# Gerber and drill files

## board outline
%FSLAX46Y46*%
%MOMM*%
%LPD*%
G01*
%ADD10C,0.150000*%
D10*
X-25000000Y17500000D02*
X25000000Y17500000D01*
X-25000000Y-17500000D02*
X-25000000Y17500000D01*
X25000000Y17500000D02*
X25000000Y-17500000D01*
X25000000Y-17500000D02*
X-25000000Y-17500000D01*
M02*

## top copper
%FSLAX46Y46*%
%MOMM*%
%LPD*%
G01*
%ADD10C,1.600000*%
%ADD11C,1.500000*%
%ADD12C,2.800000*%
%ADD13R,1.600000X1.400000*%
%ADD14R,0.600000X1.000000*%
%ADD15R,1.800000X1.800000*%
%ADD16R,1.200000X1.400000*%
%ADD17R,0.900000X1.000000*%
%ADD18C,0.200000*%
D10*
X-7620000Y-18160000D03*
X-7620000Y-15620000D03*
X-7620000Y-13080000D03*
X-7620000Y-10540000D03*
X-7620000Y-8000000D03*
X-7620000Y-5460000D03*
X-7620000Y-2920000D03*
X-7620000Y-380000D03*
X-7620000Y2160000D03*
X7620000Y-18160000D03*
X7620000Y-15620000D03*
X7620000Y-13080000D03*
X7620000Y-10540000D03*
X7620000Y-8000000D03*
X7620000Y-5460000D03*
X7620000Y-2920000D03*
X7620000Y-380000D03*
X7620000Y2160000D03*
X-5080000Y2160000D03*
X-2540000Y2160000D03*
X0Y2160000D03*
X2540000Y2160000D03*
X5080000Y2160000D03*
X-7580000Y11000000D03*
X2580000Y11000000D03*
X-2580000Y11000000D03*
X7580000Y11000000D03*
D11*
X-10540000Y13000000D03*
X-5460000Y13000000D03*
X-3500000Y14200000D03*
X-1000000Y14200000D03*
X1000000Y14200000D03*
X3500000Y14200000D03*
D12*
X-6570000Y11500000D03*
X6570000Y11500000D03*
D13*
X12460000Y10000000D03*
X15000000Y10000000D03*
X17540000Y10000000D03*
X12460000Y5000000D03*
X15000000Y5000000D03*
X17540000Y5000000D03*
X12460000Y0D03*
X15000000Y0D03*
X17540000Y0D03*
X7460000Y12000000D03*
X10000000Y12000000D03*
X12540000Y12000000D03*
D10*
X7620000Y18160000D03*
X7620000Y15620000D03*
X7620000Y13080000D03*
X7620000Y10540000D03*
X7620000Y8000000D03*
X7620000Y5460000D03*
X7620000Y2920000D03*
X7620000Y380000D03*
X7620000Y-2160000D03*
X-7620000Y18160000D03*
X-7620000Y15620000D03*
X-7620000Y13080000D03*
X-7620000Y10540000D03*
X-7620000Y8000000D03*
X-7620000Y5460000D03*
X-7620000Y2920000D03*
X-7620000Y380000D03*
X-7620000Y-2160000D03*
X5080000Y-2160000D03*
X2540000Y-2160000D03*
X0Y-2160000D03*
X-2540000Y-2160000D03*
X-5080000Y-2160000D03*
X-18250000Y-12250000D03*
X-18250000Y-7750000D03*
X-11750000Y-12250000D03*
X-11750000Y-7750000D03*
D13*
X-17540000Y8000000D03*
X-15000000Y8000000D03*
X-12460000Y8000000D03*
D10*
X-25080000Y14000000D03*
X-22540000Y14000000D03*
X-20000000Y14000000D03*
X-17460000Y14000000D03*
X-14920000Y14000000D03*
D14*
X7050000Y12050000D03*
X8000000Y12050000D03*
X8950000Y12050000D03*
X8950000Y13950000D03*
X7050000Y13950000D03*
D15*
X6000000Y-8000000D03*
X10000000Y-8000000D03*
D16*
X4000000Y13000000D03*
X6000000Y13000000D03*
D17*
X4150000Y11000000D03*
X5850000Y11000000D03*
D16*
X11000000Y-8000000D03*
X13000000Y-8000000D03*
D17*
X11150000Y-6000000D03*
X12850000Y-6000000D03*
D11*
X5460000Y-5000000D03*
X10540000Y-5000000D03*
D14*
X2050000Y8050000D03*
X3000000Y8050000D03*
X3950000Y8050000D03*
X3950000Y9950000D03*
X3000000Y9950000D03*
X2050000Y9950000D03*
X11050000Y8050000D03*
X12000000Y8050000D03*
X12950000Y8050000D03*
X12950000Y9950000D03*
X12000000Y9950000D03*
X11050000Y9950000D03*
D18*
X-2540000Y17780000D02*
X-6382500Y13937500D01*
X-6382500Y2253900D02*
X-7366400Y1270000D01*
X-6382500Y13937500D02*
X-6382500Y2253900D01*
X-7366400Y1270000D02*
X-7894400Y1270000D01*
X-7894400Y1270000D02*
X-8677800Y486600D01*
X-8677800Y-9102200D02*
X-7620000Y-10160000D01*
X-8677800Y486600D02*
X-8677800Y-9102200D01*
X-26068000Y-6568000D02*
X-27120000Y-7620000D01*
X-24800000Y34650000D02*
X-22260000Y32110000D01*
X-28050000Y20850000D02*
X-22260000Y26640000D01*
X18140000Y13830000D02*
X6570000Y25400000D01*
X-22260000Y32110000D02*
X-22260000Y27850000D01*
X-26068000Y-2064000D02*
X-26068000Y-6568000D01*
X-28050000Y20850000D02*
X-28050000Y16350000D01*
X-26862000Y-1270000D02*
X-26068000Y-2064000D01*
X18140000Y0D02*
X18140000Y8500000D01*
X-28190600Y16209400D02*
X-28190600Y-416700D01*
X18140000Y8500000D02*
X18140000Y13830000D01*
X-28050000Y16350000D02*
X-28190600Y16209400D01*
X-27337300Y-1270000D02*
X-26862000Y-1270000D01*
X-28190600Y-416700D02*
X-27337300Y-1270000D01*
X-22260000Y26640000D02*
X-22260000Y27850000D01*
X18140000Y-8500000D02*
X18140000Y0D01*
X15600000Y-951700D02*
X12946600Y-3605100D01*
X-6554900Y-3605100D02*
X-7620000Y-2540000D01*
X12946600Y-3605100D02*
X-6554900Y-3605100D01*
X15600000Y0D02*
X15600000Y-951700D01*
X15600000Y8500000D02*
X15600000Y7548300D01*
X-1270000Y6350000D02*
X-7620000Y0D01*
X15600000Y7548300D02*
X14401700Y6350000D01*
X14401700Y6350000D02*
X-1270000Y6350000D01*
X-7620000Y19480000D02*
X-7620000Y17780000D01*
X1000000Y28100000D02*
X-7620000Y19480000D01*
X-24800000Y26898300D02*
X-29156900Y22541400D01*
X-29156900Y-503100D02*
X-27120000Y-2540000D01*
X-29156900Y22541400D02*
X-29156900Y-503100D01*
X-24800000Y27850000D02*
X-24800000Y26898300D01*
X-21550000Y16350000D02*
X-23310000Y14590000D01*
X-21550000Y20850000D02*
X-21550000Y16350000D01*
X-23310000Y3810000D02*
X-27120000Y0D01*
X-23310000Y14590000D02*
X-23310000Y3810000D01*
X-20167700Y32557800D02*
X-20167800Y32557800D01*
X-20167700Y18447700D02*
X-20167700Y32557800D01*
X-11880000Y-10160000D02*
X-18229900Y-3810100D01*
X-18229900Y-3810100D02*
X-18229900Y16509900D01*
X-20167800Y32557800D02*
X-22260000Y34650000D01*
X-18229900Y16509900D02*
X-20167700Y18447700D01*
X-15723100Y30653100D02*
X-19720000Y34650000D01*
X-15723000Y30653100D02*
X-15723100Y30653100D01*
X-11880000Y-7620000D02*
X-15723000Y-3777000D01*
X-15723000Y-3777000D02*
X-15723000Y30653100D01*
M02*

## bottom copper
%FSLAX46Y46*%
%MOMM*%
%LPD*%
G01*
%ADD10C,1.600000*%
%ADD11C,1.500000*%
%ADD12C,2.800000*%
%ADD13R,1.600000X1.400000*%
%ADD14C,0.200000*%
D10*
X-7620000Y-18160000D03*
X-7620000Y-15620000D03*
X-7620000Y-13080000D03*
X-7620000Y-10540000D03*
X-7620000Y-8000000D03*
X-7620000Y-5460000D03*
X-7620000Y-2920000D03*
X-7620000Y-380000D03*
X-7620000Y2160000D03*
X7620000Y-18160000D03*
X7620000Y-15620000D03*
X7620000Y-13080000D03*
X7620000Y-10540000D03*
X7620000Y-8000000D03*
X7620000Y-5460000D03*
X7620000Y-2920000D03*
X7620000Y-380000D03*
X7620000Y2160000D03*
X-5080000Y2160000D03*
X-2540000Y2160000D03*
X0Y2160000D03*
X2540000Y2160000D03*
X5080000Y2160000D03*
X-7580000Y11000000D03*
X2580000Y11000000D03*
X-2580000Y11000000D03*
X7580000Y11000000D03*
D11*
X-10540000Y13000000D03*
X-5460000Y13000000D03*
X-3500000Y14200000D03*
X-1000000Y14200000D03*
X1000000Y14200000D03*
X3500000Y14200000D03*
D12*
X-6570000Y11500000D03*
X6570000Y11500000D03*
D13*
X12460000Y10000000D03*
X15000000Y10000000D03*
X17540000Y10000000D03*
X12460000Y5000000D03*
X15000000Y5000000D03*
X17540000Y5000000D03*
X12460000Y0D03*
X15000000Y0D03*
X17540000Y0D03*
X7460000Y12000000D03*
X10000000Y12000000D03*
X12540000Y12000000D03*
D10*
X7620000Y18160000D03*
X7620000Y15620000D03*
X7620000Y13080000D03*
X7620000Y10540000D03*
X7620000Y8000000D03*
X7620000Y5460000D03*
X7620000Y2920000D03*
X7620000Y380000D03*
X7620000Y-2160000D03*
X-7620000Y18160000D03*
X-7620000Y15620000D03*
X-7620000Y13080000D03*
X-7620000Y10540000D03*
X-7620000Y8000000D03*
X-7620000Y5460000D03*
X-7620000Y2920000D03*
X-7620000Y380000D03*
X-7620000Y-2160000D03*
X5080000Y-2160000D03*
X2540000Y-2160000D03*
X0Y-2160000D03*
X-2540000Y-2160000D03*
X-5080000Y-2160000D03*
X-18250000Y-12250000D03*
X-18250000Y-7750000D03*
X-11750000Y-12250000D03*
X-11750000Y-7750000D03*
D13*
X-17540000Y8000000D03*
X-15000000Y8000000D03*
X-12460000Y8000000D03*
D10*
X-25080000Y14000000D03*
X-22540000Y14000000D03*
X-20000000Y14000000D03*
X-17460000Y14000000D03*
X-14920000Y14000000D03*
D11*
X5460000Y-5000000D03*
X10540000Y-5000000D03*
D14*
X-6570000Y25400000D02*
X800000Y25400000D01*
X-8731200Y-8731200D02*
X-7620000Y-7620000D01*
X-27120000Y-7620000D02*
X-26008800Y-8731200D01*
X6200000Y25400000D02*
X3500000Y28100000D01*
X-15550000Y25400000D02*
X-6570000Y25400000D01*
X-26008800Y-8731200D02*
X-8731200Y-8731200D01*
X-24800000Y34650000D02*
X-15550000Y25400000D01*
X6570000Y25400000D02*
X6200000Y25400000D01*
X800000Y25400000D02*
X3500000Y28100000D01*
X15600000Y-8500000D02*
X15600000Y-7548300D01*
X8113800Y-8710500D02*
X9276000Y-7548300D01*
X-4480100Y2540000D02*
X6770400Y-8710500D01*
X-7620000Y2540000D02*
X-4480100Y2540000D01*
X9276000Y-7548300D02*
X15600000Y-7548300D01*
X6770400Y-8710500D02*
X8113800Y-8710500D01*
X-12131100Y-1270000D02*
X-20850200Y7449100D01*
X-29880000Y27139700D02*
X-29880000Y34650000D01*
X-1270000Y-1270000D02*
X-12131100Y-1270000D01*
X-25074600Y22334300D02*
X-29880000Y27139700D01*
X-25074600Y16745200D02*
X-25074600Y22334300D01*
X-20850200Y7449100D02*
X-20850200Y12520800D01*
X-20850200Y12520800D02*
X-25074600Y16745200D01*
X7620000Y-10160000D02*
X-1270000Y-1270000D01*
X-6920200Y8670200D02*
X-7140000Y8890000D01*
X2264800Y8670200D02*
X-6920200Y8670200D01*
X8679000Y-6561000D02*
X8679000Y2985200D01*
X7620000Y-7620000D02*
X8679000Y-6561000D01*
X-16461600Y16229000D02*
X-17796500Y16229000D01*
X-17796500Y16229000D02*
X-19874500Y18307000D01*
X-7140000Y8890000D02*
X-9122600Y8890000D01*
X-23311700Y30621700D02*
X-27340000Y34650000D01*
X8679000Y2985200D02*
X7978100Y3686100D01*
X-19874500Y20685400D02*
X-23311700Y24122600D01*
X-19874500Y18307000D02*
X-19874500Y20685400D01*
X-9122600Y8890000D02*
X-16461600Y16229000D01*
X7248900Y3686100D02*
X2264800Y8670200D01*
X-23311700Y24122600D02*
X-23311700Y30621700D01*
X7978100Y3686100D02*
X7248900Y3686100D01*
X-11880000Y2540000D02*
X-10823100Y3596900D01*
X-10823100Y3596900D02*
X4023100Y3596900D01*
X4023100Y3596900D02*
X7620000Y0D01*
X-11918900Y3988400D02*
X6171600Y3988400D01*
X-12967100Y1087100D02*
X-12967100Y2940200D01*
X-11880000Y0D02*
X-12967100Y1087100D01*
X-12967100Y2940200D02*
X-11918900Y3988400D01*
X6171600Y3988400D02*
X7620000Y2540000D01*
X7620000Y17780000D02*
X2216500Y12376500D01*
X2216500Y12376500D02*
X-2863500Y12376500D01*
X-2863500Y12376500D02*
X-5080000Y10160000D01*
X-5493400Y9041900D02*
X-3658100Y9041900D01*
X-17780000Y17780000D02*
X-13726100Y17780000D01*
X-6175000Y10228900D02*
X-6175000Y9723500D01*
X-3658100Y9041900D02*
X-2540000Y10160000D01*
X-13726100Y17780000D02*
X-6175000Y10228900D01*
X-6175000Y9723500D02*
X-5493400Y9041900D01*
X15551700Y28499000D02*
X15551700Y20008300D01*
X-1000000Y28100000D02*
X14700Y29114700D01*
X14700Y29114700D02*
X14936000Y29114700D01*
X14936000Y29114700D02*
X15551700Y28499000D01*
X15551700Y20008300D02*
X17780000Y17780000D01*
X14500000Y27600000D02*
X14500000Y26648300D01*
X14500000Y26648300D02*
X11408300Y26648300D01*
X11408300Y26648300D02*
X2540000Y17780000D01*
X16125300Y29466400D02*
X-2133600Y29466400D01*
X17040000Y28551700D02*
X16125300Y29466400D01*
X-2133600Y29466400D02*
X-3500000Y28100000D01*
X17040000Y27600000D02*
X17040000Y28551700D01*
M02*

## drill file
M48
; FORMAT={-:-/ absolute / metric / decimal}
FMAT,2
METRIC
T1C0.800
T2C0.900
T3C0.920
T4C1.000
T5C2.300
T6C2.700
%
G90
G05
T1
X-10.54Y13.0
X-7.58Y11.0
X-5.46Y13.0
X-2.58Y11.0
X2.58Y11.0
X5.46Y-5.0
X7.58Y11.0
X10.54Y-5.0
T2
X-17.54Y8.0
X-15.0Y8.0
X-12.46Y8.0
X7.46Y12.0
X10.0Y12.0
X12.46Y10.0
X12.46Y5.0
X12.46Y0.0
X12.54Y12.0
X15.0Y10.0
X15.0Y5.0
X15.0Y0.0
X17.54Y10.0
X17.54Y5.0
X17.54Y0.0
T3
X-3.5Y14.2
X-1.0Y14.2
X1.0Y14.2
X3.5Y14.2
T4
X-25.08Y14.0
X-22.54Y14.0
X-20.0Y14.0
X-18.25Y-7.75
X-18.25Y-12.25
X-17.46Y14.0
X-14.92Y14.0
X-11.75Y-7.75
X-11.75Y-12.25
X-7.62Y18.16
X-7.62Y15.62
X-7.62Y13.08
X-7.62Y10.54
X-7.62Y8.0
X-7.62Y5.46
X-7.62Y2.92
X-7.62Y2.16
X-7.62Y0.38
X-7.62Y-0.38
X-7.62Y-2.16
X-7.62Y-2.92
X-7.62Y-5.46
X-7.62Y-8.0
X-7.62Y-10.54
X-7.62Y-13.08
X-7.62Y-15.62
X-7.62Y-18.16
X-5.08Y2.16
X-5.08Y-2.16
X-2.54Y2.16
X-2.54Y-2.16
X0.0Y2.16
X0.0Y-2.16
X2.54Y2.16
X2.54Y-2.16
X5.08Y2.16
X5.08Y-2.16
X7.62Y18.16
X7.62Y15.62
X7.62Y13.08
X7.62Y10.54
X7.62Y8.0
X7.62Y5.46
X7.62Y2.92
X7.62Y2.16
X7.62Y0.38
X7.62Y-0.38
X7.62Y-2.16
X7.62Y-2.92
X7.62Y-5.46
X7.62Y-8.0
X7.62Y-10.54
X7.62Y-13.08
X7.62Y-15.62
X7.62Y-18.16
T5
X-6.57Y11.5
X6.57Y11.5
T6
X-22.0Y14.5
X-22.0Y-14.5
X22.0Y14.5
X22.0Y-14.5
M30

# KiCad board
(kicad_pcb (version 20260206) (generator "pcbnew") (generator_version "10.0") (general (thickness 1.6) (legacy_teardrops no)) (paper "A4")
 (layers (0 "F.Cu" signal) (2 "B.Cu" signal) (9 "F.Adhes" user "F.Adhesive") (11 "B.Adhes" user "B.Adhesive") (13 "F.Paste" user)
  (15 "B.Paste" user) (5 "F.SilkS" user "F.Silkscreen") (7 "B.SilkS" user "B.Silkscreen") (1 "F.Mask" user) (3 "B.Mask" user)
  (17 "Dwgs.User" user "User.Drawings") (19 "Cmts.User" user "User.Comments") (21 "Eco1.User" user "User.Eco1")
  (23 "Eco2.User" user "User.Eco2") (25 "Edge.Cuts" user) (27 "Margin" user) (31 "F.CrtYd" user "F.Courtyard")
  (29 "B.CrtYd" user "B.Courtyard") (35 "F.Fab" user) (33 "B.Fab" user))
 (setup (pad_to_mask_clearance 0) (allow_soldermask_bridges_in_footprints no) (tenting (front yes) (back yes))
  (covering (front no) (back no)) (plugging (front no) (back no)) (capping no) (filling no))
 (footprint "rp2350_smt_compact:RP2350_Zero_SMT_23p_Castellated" (layer "F.Cu") (at 0 8)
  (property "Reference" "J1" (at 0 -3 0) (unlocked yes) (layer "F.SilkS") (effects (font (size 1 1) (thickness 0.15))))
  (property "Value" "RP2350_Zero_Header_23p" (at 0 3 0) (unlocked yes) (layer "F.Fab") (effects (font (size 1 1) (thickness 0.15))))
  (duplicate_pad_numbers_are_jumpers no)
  (pad "1" thru_hole circle (at -7.62 10.16) (size 1.6 1.6) (drill 1) (layers "*.Cu" "*.Mask") (remove_unused_layers no) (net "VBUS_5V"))
  (pad "2" thru_hole circle (at -7.62 7.62) (size 1.6 1.6) (drill 1) (layers "*.Cu" "*.Mask") (remove_unused_layers no) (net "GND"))
  (pad "3" thru_hole circle (at -7.62 5.08) (size 1.6 1.6) (drill 1) (layers "*.Cu" "*.Mask") (remove_unused_layers no))
  (pad "4" thru_hole circle (at -7.62 2.54) (size 1.6 1.6) (drill 1) (layers "*.Cu" "*.Mask") (remove_unused_layers no)
   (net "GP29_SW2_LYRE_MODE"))
  (pad "5" thru_hole circle (at -7.62 0) (size 1.6 1.6) (drill 1) (layers "*.Cu" "*.Mask") (remove_unused_layers no)
   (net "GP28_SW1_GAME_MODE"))
  (pad "6" thru_hole circle (at -7.62 -2.54) (size 1.6 1.6) (drill 1) (layers "*.Cu" "*.Mask") (remove_unused_layers no)
   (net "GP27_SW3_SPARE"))
  (pad "7" thru_hole circle (at -7.62 -5.08) (size 1.6 1.6) (drill 1) (layers "*.Cu" "*.Mask") (remove_unused_layers no))
  (pad "8" thru_hole circle (at -7.62 -7.62) (size 1.6 1.6) (drill 1) (layers "*.Cu" "*.Mask") (remove_unused_layers no))
  (pad "9" thru_hole circle (at -7.62 -10.16) (size 1.6 1.6) (drill 1) (layers "*.Cu" "*.Mask") (remove_unused_layers no))
  (pad "10" thru_hole circle (at 7.62 10.16) (size 1.6 1.6) (drill 1) (layers "*.Cu" "*.Mask") (remove_unused_layers no)
   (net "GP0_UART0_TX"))
  (pad "11" thru_hole circle (at 7.62 7.62) (size 1.6 1.6) (drill 1) (layers "*.Cu" "*.Mask") (remove_unused_layers no) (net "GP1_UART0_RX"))
  (pad "12" thru_hole circle (at 7.62 5.08) (size 1.6 1.6) (drill 1) (layers "*.Cu" "*.Mask") (remove_unused_layers no))
  (pad "13" thru_hole circle (at 7.62 2.54) (size 1.6 1.6) (drill 1) (layers "*.Cu" "*.Mask") (remove_unused_layers no))
  (pad "14" thru_hole circle (at 7.62 0) (size 1.6 1.6) (drill 1) (layers "*.Cu" "*.Mask") (remove_unused_layers no) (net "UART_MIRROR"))
  (pad "15" thru_hole circle (at 7.62 -2.54) (size 1.6 1.6) (drill 1) (layers "*.Cu" "*.Mask") (remove_unused_layers no)
   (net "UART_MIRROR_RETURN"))
  (pad "16" thru_hole circle (at 7.62 -5.08) (size 1.6 1.6) (drill 1) (layers "*.Cu" "*.Mask") (remove_unused_layers no))
  (pad "17" thru_hole circle (at 7.62 -7.62) (size 1.6 1.6) (drill 1) (layers "*.Cu" "*.Mask") (remove_unused_layers no))
  (pad "18" thru_hole circle (at 7.62 -10.16) (size 1.6 1.6) (drill 1) (layers "*.Cu" "*.Mask") (remove_unused_layers no))
  (pad "19" thru_hole circle (at -5.08 -10.16) (size 1.6 1.6) (drill 1) (layers "*.Cu" "*.Mask") (remove_unused_layers no)
   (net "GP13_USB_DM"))
  (pad "20" thru_hole circle (at -2.54 -10.16) (size 1.6 1.6) (drill 1) (layers "*.Cu" "*.Mask") (remove_unused_layers no)
   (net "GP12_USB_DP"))
  (pad "21" thru_hole circle (at 0 -10.16) (size 1.6 1.6) (drill 1) (layers "*.Cu" "*.Mask") (remove_unused_layers no))
  (pad "22" thru_hole circle (at 2.54 -10.16) (size 1.6 1.6) (drill 1) (layers "*.Cu" "*.Mask") (remove_unused_layers no))
  (pad "23" thru_hole circle (at 5.08 -10.16) (size 1.6 1.6) (drill 1) (layers "*.Cu" "*.Mask") (remove_unused_layers no)))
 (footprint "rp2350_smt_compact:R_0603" (layer "F.Cu") (at -2.5 -11)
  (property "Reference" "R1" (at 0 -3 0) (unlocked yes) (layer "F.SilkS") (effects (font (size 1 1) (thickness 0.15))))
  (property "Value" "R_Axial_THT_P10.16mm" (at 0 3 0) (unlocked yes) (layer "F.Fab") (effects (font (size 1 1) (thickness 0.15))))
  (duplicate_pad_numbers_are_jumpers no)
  (pad "1" thru_hole circle (at -5.08 0) (size 1.6 1.6) (drill 0.8) (layers "*.Cu" "*.Mask") (remove_unused_layers no) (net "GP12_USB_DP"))
  (pad "2" thru_hole circle (at 5.08 0) (size 1.6 1.6) (drill 0.8) (layers "*.Cu" "*.Mask") (remove_unused_layers no) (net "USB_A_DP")))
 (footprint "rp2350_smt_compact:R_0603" (layer "F.Cu") (at 2.5 -11)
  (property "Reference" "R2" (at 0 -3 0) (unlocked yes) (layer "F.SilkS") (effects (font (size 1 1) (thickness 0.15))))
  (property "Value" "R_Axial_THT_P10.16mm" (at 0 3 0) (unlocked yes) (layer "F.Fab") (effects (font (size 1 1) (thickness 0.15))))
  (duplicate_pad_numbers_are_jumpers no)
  (pad "1" thru_hole circle (at -5.08 0) (size 1.6 1.6) (drill 0.8) (layers "*.Cu" "*.Mask") (remove_unused_layers no) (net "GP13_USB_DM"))
  (pad "2" thru_hole circle (at 5.08 0) (size 1.6 1.6) (drill 0.8) (layers "*.Cu" "*.Mask") (remove_unused_layers no) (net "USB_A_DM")))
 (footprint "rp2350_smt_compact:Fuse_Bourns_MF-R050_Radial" (layer "F.Cu") (at -8 -13)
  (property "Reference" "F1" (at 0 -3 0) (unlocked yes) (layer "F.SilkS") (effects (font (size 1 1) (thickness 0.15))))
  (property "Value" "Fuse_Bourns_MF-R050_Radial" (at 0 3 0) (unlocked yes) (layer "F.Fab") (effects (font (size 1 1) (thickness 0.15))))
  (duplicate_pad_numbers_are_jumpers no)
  (pad "1" thru_hole circle (at -2.54 0) (size 1.5 1.5) (drill 0.8) (layers "*.Cu" "*.Mask") (remove_unused_layers no) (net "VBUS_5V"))
  (pad "2" thru_hole circle (at 2.54 0) (size 1.5 1.5) (drill 0.8) (layers "*.Cu" "*.Mask") (remove_unused_layers no) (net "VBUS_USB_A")))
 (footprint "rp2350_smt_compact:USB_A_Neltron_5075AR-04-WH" (layer "F.Cu") (at 0 -14.2)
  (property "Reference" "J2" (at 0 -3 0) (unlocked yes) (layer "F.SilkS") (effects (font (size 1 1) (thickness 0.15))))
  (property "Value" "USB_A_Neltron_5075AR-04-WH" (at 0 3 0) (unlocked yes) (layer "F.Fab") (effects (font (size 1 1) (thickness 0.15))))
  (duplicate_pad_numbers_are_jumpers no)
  (pad "1" thru_hole circle (at -3.5 0) (size 1.5 1.5) (drill 0.92) (layers "*.Cu" "*.Mask") (remove_unused_layers no) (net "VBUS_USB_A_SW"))
  (pad "2" thru_hole circle (at -1 0) (size 1.5 1.5) (drill 0.92) (layers "*.Cu" "*.Mask") (remove_unused_layers no) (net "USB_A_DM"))
  (pad "3" thru_hole circle (at 1 0) (size 1.5 1.5) (drill 0.92) (layers "*.Cu" "*.Mask") (remove_unused_layers no) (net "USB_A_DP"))
  (pad "4" thru_hole circle (at 3.5 0) (size 1.5 1.5) (drill 0.92) (layers "*.Cu" "*.Mask") (remove_unused_layers no) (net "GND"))
  (pad "5" thru_hole circle (at -6.57 2.7) (size 2.8 2.8) (drill 2.3) (layers "*.Cu" "*.Mask") (remove_unused_layers no) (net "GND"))
  (pad "6" thru_hole circle (at 6.57 2.7) (size 2.8 2.8) (drill 2.3) (layers "*.Cu" "*.Mask") (remove_unused_layers no) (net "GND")))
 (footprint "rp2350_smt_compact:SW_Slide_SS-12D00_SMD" (layer "F.Cu") (at 15 -10)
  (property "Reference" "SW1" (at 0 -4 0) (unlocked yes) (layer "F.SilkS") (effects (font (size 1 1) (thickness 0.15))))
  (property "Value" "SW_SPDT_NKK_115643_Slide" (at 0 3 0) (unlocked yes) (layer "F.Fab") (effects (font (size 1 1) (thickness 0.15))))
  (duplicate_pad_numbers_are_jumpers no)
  (pad "1" thru_hole rect (at -2.54 0) (size 1.6 1.4) (drill 0.9) (layers "*.Cu" "*.Mask") (remove_unused_layers no))
  (pad "2" thru_hole rect (at 0 0) (size 1.6 1.4) (drill 0.9) (layers "*.Cu" "*.Mask") (remove_unused_layers no) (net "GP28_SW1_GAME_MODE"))
  (pad "3" thru_hole rect (at 2.54 0) (size 1.6 1.4) (drill 0.9) (layers "*.Cu" "*.Mask") (remove_unused_layers no) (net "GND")))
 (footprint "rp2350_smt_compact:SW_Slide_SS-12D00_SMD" (layer "F.Cu") (at 15 -5)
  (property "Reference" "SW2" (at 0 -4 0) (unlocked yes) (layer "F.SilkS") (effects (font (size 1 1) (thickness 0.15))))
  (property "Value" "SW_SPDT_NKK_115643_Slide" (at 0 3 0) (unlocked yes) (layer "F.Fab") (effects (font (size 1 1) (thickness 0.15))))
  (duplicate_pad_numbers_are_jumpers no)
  (pad "1" thru_hole rect (at -2.54 0) (size 1.6 1.4) (drill 0.9) (layers "*.Cu" "*.Mask") (remove_unused_layers no))
  (pad "2" thru_hole rect (at 0 0) (size 1.6 1.4) (drill 0.9) (layers "*.Cu" "*.Mask") (remove_unused_layers no) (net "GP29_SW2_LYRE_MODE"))
  (pad "3" thru_hole rect (at 2.54 0) (size 1.6 1.4) (drill 0.9) (layers "*.Cu" "*.Mask") (remove_unused_layers no) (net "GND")))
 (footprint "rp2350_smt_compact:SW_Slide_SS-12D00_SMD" (layer "F.Cu") (at 15 0)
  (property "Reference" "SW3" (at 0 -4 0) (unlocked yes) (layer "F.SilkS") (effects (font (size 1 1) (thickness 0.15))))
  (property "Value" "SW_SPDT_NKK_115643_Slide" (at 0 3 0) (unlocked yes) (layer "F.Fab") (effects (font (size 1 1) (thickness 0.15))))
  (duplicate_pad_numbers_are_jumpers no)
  (pad "1" thru_hole rect (at -2.54 0) (size 1.6 1.4) (drill 0.9) (layers "*.Cu" "*.Mask") (remove_unused_layers no))
  (pad "2" thru_hole rect (at 0 0) (size 1.6 1.4) (drill 0.9) (layers "*.Cu" "*.Mask") (remove_unused_layers no) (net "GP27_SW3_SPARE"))
  (pad "3" thru_hole rect (at 2.54 0) (size 1.6 1.4) (drill 0.9) (layers "*.Cu" "*.Mask") (remove_unused_layers no) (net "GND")))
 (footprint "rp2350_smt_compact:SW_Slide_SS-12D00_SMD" (layer "F.Cu") (at 10 -12)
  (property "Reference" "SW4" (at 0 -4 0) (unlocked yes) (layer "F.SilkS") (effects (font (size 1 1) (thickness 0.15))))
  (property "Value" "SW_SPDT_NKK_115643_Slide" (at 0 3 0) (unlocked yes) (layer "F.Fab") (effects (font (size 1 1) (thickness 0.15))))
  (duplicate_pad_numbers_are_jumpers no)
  (pad "1" thru_hole rect (at -2.54 0) (size 1.6 1.4) (drill 0.9) (layers "*.Cu" "*.Mask") (remove_unused_layers no))
  (pad "2" thru_hole rect (at 0 0) (size 1.6 1.4) (drill 0.9) (layers "*.Cu" "*.Mask") (remove_unused_layers no) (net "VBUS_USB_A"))
  (pad "3" thru_hole rect (at 2.54 0) (size 1.6 1.4) (drill 0.9) (layers "*.Cu" "*.Mask") (remove_unused_layers no) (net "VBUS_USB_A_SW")))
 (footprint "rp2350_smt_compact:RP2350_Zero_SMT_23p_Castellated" (layer "F.Cu") (at 0 -8 180)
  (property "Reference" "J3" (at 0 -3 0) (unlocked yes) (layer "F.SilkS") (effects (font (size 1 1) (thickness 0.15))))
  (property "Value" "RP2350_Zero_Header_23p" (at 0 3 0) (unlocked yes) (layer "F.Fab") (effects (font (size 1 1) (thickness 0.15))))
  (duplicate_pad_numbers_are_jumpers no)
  (pad "1" thru_hole circle (at -7.62 10.16) (size 1.6 1.6) (drill 1) (layers "*.Cu" "*.Mask") (remove_unused_layers no))
  (pad "2" thru_hole circle (at -7.62 7.62) (size 1.6 1.6) (drill 1) (layers "*.Cu" "*.Mask") (remove_unused_layers no) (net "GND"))
  (pad "3" thru_hole circle (at -7.62 5.08) (size 1.6 1.6) (drill 1) (layers "*.Cu" "*.Mask") (remove_unused_layers no))
  (pad "4" thru_hole circle (at -7.62 2.54) (size 1.6 1.6) (drill 1) (layers "*.Cu" "*.Mask") (remove_unused_layers no)
   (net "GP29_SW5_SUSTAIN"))
  (pad "5" thru_hole circle (at -7.62 0) (size 1.6 1.6) (drill 1) (layers "*.Cu" "*.Mask") (remove_unused_layers no) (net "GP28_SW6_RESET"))
  (pad "6" thru_hole circle (at -7.62 -2.54) (size 1.6 1.6) (drill 1) (layers "*.Cu" "*.Mask") (remove_unused_layers no))
  (pad "7" thru_hole circle (at -7.62 -5.08) (size 1.6 1.6) (drill 1) (layers "*.Cu" "*.Mask") (remove_unused_layers no))
  (pad "8" thru_hole circle (at -7.62 -7.62) (size 1.6 1.6) (drill 1) (layers "*.Cu" "*.Mask") (remove_unused_layers no))
  (pad "9" thru_hole circle (at -7.62 -10.16) (size 1.6 1.6) (drill 1) (layers "*.Cu" "*.Mask") (remove_unused_layers no))
  (pad "10" thru_hole circle (at 7.62 10.16) (size 1.6 1.6) (drill 1) (layers "*.Cu" "*.Mask") (remove_unused_layers no)
   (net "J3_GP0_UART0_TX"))
  (pad "11" thru_hole circle (at 7.62 7.62) (size 1.6 1.6) (drill 1) (layers "*.Cu" "*.Mask") (remove_unused_layers no)
   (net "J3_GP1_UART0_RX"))
  (pad "12" thru_hole circle (at 7.62 5.08) (size 1.6 1.6) (drill 1) (layers "*.Cu" "*.Mask") (remove_unused_layers no))
  (pad "13" thru_hole circle (at 7.62 2.54) (size 1.6 1.6) (drill 1) (layers "*.Cu" "*.Mask") (remove_unused_layers no))
  (pad "14" thru_hole circle (at 7.62 0) (size 1.6 1.6) (drill 1) (layers "*.Cu" "*.Mask") (remove_unused_layers no)
   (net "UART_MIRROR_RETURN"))
  (pad "15" thru_hole circle (at 7.62 -2.54) (size 1.6 1.6) (drill 1) (layers "*.Cu" "*.Mask") (remove_unused_layers no) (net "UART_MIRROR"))
  (pad "16" thru_hole circle (at 7.62 -5.08) (size 1.6 1.6) (drill 1) (layers "*.Cu" "*.Mask") (remove_unused_layers no))
  (pad "17" thru_hole circle (at 7.62 -7.62) (size 1.6 1.6) (drill 1) (layers "*.Cu" "*.Mask") (remove_unused_layers no))
  (pad "18" thru_hole circle (at 7.62 -10.16) (size 1.6 1.6) (drill 1) (layers "*.Cu" "*.Mask") (remove_unused_layers no))
  (pad "19" thru_hole circle (at -5.08 -10.16) (size 1.6 1.6) (drill 1) (layers "*.Cu" "*.Mask") (remove_unused_layers no))
  (pad "20" thru_hole circle (at -2.54 -10.16) (size 1.6 1.6) (drill 1) (layers "*.Cu" "*.Mask") (remove_unused_layers no))
  (pad "21" thru_hole circle (at 0 -10.16) (size 1.6 1.6) (drill 1) (layers "*.Cu" "*.Mask") (remove_unused_layers no))
  (pad "22" thru_hole circle (at 2.54 -10.16) (size 1.6 1.6) (drill 1) (layers "*.Cu" "*.Mask") (remove_unused_layers no))
  (pad "23" thru_hole circle (at 5.08 -10.16) (size 1.6 1.6) (drill 1) (layers "*.Cu" "*.Mask") (remove_unused_layers no)))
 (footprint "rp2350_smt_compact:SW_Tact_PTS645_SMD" (layer "F.Cu") (at -15 10)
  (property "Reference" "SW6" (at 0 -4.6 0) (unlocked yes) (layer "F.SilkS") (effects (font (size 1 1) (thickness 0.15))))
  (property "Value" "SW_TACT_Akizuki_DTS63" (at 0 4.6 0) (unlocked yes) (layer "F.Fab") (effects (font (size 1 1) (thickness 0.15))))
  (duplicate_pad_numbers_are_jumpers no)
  (pad "1" thru_hole circle (at -3.25 2.25) (size 1.6 1.6) (drill 1) (layers "*.Cu" "*.Mask") (remove_unused_layers no) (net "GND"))
  (pad "2" thru_hole circle (at -3.25 -2.25) (size 1.6 1.6) (drill 1) (layers "*.Cu" "*.Mask") (remove_unused_layers no) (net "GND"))
  (pad "3" thru_hole circle (at 3.25 2.25) (size 1.6 1.6) (drill 1) (layers "*.Cu" "*.Mask") (remove_unused_layers no)
   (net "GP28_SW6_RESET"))
  (pad "4" thru_hole circle (at 3.25 -2.25) (size 1.6 1.6) (drill 1) (layers "*.Cu" "*.Mask") (remove_unused_layers no)
   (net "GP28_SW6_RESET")))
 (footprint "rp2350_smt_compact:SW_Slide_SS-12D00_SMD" (layer "F.Cu") (at -15 -8)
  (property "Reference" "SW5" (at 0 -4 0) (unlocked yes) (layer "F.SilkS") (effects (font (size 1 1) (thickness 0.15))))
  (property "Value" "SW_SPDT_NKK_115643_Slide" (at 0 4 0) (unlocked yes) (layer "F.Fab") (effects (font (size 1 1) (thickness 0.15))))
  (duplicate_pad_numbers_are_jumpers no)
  (pad "1" thru_hole rect (at -2.54 0) (size 1.6 1.4) (drill 0.9) (layers "*.Cu" "*.Mask") (remove_unused_layers no))
  (pad "2" thru_hole rect (at 0 0) (size 1.6 1.4) (drill 0.9) (layers "*.Cu" "*.Mask") (remove_unused_layers no) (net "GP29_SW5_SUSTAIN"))
  (pad "3" thru_hole rect (at 2.54 0) (size 1.6 1.4) (drill 0.9) (layers "*.Cu" "*.Mask") (remove_unused_layers no) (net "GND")))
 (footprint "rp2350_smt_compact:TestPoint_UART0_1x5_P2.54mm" (layer "F.Cu") (at -20 -14)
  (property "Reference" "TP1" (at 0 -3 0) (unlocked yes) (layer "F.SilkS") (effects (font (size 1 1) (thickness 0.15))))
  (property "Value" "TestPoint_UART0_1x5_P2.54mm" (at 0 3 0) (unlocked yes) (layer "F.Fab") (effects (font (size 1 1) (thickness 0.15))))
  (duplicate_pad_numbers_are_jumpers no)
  (pad "1" thru_hole circle (at -5.08 0) (size 1.6 1.6) (drill 1) (layers "*.Cu" "*.Mask") (remove_unused_layers no) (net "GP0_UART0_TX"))
  (pad "2" thru_hole circle (at -2.54 0) (size 1.6 1.6) (drill 1) (layers "*.Cu" "*.Mask") (remove_unused_layers no) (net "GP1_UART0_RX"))
  (pad "3" thru_hole circle (at 0 0) (size 1.6 1.6) (drill 1) (layers "*.Cu" "*.Mask") (remove_unused_layers no) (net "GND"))
  (pad "4" thru_hole circle (at 2.54 0) (size 1.6 1.6) (drill 1) (layers "*.Cu" "*.Mask") (remove_unused_layers no) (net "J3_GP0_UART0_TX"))
  (pad "5" thru_hole circle (at 5.08 0) (size 1.6 1.6) (drill 1) (layers "*.Cu" "*.Mask") (remove_unused_layers no) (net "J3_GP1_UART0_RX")))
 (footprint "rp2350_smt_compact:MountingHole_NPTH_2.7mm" (layer "F.Cu") (at -22 14.5)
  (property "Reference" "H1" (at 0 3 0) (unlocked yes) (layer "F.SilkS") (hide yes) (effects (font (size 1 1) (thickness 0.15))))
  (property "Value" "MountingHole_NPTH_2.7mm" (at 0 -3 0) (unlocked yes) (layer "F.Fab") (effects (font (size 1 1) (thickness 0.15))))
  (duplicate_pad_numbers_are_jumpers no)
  (pad "" np_thru_hole circle (at 0 0) (size 2.7 2.7) (drill 2.7) (layers "*.Cu" "*.Mask")))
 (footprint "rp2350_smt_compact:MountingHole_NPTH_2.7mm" (layer "F.Cu") (at 22 -14.5)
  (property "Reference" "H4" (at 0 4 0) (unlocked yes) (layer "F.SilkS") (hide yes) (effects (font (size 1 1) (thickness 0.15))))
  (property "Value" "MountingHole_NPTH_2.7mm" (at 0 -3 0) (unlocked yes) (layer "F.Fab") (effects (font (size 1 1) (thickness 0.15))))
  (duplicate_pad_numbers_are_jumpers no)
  (pad "" np_thru_hole circle (at 0 0) (size 2.7 2.7) (drill 2.7) (layers "*.Cu" "*.Mask")))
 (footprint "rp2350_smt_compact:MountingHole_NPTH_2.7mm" (layer "F.Cu") (at 22 14.5)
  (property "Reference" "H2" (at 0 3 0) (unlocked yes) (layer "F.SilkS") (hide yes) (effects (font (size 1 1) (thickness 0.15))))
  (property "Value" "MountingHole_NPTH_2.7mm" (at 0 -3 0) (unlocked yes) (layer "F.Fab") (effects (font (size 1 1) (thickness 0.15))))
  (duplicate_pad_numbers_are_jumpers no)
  (pad "" np_thru_hole circle (at 0 0) (size 2.7 2.7) (drill 2.7) (layers "*.Cu" "*.Mask")))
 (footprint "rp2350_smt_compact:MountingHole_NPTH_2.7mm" (layer "F.Cu") (at -22 -14.5)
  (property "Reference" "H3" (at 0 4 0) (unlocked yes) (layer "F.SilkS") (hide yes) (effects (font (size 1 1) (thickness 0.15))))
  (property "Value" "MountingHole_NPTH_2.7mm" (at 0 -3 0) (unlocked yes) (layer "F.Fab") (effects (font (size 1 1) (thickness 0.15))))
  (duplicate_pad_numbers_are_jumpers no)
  (pad "" np_thru_hole circle (at 0 0) (size 2.7 2.7) (drill 2.7) (layers "*.Cu" "*.Mask")))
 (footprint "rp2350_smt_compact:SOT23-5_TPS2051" (layer "F.Cu") (at 8 -13)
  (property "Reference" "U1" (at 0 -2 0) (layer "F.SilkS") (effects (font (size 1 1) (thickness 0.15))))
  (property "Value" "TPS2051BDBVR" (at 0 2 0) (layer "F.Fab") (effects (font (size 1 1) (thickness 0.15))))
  (pad "1" smd rect (at -0.95 0.95) (size 0.6 1) (layers "F.Cu" "F.Paste" "F.Mask"))
  (pad "2" smd rect (at 0 0.95) (size 0.6 1) (layers "F.Cu" "F.Paste" "F.Mask"))
  (pad "3" smd rect (at 0.95 0.95) (size 0.6 1) (layers "F.Cu" "F.Paste" "F.Mask"))
  (pad "4" smd rect (at 0.95 -0.95) (size 0.6 1) (layers "F.Cu" "F.Paste" "F.Mask"))
  (pad "5" smd rect (at -0.95 -0.95) (size 0.6 1) (layers "F.Cu" "F.Paste" "F.Mask")))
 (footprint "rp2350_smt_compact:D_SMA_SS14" (layer "F.Cu") (at 8 8)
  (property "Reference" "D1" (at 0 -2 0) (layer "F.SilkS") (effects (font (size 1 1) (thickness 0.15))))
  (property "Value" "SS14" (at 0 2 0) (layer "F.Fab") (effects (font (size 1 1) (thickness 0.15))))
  (pad "1" smd rect (at -2 0) (size 1.8 1.8) (layers "F.Cu" "F.Paste" "F.Mask"))
  (pad "2" smd rect (at 2 0) (size 1.8 1.8) (layers "F.Cu" "F.Paste" "F.Mask")))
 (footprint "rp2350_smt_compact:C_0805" (layer "F.Cu") (at 5 -13)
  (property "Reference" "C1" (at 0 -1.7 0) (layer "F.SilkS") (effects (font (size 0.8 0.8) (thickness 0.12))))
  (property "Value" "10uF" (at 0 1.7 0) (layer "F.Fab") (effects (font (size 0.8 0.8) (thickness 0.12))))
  (pad "1" smd rect (at -1 0) (size 1.2 1.4) (layers "F.Cu" "F.Paste" "F.Mask"))
  (pad "2" smd rect (at 1 0) (size 1.2 1.4) (layers "F.Cu" "F.Paste" "F.Mask")))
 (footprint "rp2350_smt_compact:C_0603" (layer "F.Cu") (at 5 -11)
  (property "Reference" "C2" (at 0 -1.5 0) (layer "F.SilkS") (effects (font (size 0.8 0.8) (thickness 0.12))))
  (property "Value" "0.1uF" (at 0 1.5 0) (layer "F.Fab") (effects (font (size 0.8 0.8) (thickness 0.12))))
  (pad "1" smd rect (at -0.85 0) (size 0.9 1) (layers "F.Cu" "F.Paste" "F.Mask"))
  (pad "2" smd rect (at 0.85 0) (size 0.9 1) (layers "F.Cu" "F.Paste" "F.Mask")))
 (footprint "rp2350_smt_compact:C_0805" (layer "F.Cu") (at 12 8)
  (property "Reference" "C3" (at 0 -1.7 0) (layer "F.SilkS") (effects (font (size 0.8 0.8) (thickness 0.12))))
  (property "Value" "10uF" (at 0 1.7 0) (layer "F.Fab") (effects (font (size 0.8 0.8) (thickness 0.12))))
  (pad "1" smd rect (at -1 0) (size 1.2 1.4) (layers "F.Cu" "F.Paste" "F.Mask"))
  (pad "2" smd rect (at 1 0) (size 1.2 1.4) (layers "F.Cu" "F.Paste" "F.Mask")))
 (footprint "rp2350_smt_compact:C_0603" (layer "F.Cu") (at 12 6)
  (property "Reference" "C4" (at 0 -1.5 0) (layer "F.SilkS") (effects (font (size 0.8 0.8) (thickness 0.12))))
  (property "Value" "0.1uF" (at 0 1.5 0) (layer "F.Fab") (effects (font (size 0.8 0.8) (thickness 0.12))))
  (pad "1" smd rect (at -0.85 0) (size 0.9 1) (layers "F.Cu" "F.Paste" "F.Mask"))
  (pad "2" smd rect (at 0.85 0) (size 0.9 1) (layers "F.Cu" "F.Paste" "F.Mask")))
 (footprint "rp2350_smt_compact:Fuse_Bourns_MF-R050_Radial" (layer "F.Cu") (at 8 5)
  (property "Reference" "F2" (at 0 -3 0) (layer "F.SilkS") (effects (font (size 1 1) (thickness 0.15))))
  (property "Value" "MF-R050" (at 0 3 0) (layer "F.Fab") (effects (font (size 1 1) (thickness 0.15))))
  (pad "1" thru_hole circle (at -2.54 0) (size 1.5 1.5) (drill 0.8) (layers "*.Cu" "*.Mask"))
  (pad "2" thru_hole circle (at 2.54 0) (size 1.5 1.5) (drill 0.8) (layers "*.Cu" "*.Mask")))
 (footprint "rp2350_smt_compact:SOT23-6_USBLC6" (layer "F.Cu") (at 3 -9)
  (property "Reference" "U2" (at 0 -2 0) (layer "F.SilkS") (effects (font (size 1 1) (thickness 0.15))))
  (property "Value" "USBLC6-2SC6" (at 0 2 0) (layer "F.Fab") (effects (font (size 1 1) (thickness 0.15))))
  (pad "1" smd rect (at -0.95 0.95) (size 0.6 1) (layers "F.Cu" "F.Paste" "F.Mask"))
  (pad "2" smd rect (at 0 0.95) (size 0.6 1) (layers "F.Cu" "F.Paste" "F.Mask"))
  (pad "3" smd rect (at 0.95 0.95) (size 0.6 1) (layers "F.Cu" "F.Paste" "F.Mask"))
  (pad "4" smd rect (at 0.95 -0.95) (size 0.6 1) (layers "F.Cu" "F.Paste" "F.Mask"))
  (pad "5" smd rect (at 0 -0.95) (size 0.6 1) (layers "F.Cu" "F.Paste" "F.Mask"))
  (pad "6" smd rect (at -0.95 -0.95) (size 0.6 1) (layers "F.Cu" "F.Paste" "F.Mask")))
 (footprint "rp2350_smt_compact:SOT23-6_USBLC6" (layer "F.Cu") (at 12 -9)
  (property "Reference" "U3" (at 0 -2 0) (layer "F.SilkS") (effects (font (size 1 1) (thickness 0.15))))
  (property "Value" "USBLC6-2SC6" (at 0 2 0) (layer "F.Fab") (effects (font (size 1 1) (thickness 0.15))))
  (pad "1" smd rect (at -0.95 0.95) (size 0.6 1) (layers "F.Cu" "F.Paste" "F.Mask"))
  (pad "2" smd rect (at 0 0.95) (size 0.6 1) (layers "F.Cu" "F.Paste" "F.Mask"))
  (pad "3" smd rect (at 0.95 0.95) (size 0.6 1) (layers "F.Cu" "F.Paste" "F.Mask"))
  (pad "4" smd rect (at 0.95 -0.95) (size 0.6 1) (layers "F.Cu" "F.Paste" "F.Mask"))
  (pad "5" smd rect (at 0 -0.95) (size 0.6 1) (layers "F.Cu" "F.Paste" "F.Mask"))
  (pad "6" smd rect (at -0.95 -0.95) (size 0.6 1) (layers "F.Cu" "F.Paste" "F.Mask")))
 (gr_line (start -25 -17.5) (end 25 -17.5) (stroke (width 0.15) (type solid)) (layer "Edge.Cuts"))
 (gr_line (start -25 17.5) (end -25 -17.5) (stroke (width 0.15) (type solid)) (layer "Edge.Cuts"))
 (gr_line (start 25 -17.5) (end 25 17.5) (stroke (width 0.15) (type solid)) (layer "Edge.Cuts"))
 (gr_line (start 25 17.5) (end -25 17.5) (stroke (width 0.15) (type solid)) (layer "Edge.Cuts"))
 (segment (start -2.54 -17.78) (end -6.3825 -13.9375) (width 0.2) (layer "F.Cu") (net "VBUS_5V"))
 (segment (start -6.3825 -2.2539) (end -7.3664 -1.27) (width 0.2) (layer "F.Cu") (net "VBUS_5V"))
 (segment (start -6.3825 -13.9375) (end -6.3825 -2.2539) (width 0.2) (layer "F.Cu") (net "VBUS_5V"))
 (segment (start -7.3664 -1.27) (end -7.8944 -1.27) (width 0.2) (layer "F.Cu") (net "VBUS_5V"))
 (segment (start -7.8944 -1.27) (end -8.6778 -0.4866) (width 0.2) (layer "F.Cu") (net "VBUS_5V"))
 (segment (start -8.6778 9.1022) (end -7.62 10.16) (width 0.2) (layer "F.Cu") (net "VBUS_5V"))
 (segment (start -8.6778 -0.4866) (end -8.6778 9.1022) (width 0.2) (layer "F.Cu") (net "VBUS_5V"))
 (segment (start -26.068 6.568) (end -27.12 7.62) (width 0.2) (layer "F.Cu") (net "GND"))
 (segment (start -24.8 -34.65) (end -22.26 -32.11) (width 0.2) (layer "F.Cu") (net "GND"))
 (segment (start -28.05 -20.85) (end -22.26 -26.64) (width 0.2) (layer "F.Cu") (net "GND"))
 (segment (start 18.14 -13.83) (end 6.57 -25.4) (width 0.2) (layer "F.Cu") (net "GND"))
 (segment (start -22.26 -32.11) (end -22.26 -27.85) (width 0.2) (layer "F.Cu") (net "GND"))
 (segment (start -26.068 2.064) (end -26.068 6.568) (width 0.2) (layer "F.Cu") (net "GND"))
 (segment (start -28.05 -20.85) (end -28.05 -16.35) (width 0.2) (layer "F.Cu") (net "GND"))
 (segment (start -26.862 1.27) (end -26.068 2.064) (width 0.2) (layer "F.Cu") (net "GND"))
 (segment (start 18.14 0) (end 18.14 -8.5) (width 0.2) (layer "F.Cu") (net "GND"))
 (segment (start -28.1906 -16.2094) (end -28.1906 0.4167) (width 0.2) (layer "F.Cu") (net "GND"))
 (segment (start 18.14 -8.5) (end 18.14 -13.83) (width 0.2) (layer "F.Cu") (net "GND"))
 (segment (start -28.05 -16.35) (end -28.1906 -16.2094) (width 0.2) (layer "F.Cu") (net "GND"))
 (segment (start -27.3373 1.27) (end -26.862 1.27) (width 0.2) (layer "F.Cu") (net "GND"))
 (segment (start -28.1906 0.4167) (end -27.3373 1.27) (width 0.2) (layer "F.Cu") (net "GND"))
 (segment (start -22.26 -26.64) (end -22.26 -27.85) (width 0.2) (layer "F.Cu") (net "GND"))
 (segment (start 18.14 8.5) (end 18.14 0) (width 0.2) (layer "F.Cu") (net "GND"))
 (segment (start -6.57 -25.4) (end 0.8 -25.4) (width 0.2) (layer "B.Cu") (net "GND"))
 (segment (start -8.7312 8.7312) (end -7.62 7.62) (width 0.2) (layer "B.Cu") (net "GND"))
 (segment (start -27.12 7.62) (end -26.0088 8.7312) (width 0.2) (layer "B.Cu") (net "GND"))
 (segment (start 6.2 -25.4) (end 3.5 -28.1) (width 0.2) (layer "B.Cu") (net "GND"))
 (segment (start -15.55 -25.4) (end -6.57 -25.4) (width 0.2) (layer "B.Cu") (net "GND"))
 (segment (start -26.0088 8.7312) (end -8.7312 8.7312) (width 0.2) (layer "B.Cu") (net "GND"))
 (segment (start -24.8 -34.65) (end -15.55 -25.4) (width 0.2) (layer "B.Cu") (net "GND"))
 (segment (start 6.57 -25.4) (end 6.2 -25.4) (width 0.2) (layer "B.Cu") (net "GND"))
 (segment (start 0.8 -25.4) (end 3.5 -28.1) (width 0.2) (layer "B.Cu") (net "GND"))
 (segment (start 15.6 0.9517) (end 12.9466 3.6051) (width 0.2) (layer "F.Cu") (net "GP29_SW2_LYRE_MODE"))
 (segment (start -6.5549 3.6051) (end -7.62 2.54) (width 0.2) (layer "F.Cu") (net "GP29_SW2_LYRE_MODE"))
 (segment (start 12.9466 3.6051) (end -6.5549 3.6051) (width 0.2) (layer "F.Cu") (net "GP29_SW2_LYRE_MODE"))
 (segment (start 15.6 0) (end 15.6 0.9517) (width 0.2) (layer "F.Cu") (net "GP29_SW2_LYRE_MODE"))
 (segment (start 15.6 -8.5) (end 15.6 -7.5483) (width 0.2) (layer "F.Cu") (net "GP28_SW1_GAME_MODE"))
 (segment (start -1.27 -6.35) (end -7.62 0) (width 0.2) (layer "F.Cu") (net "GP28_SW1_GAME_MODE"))
 (segment (start 15.6 -7.5483) (end 14.4017 -6.35) (width 0.2) (layer "F.Cu") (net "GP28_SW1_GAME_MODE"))
 (segment (start 14.4017 -6.35) (end -1.27 -6.35) (width 0.2) (layer "F.Cu") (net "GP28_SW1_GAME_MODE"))
 (segment (start 15.6 8.5) (end 15.6 7.5483) (width 0.2) (layer "B.Cu") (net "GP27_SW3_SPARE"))
 (segment (start 8.1138 8.7105) (end 9.276 7.5483) (width 0.2) (layer "B.Cu") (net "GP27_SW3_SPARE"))
 (segment (start -4.4801 -2.54) (end 6.7704 8.7105) (width 0.2) (layer "B.Cu") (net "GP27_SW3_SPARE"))
 (segment (start -7.62 -2.54) (end -4.4801 -2.54) (width 0.2) (layer "B.Cu") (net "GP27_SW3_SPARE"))
 (segment (start 9.276 7.5483) (end 15.6 7.5483) (width 0.2) (layer "B.Cu") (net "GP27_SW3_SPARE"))
 (segment (start 6.7704 8.7105) (end 8.1138 8.7105) (width 0.2) (layer "B.Cu") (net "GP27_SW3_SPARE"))
 (segment (start -12.1311 1.27) (end -20.8502 -7.4491) (width 0.2) (layer "B.Cu") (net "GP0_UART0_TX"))
 (segment (start -29.88 -27.1397) (end -29.88 -34.65) (width 0.2) (layer "B.Cu") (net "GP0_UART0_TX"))
 (segment (start -1.27 1.27) (end -12.1311 1.27) (width 0.2) (layer "B.Cu") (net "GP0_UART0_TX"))
 (segment (start -25.0746 -22.3343) (end -29.88 -27.1397) (width 0.2) (layer "B.Cu") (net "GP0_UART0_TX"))
 (segment (start -25.0746 -16.7452) (end -25.0746 -22.3343) (width 0.2) (layer "B.Cu") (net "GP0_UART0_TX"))
 (segment (start -20.8502 -7.4491) (end -20.8502 -12.5208) (width 0.2) (layer "B.Cu") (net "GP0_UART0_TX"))
 (segment (start -20.8502 -12.5208) (end -25.0746 -16.7452) (width 0.2) (layer "B.Cu") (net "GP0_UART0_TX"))
 (segment (start 7.62 10.16) (end -1.27 1.27) (width 0.2) (layer "B.Cu") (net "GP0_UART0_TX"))
 (segment (start -6.9202 -8.6702) (end -7.14 -8.89) (width 0.2) (layer "B.Cu") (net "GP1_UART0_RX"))
 (segment (start 2.2648 -8.6702) (end -6.9202 -8.6702) (width 0.2) (layer "B.Cu") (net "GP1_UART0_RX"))
 (segment (start 8.679 6.561) (end 8.679 -2.9852) (width 0.2) (layer "B.Cu") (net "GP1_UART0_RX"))
 (segment (start 7.62 7.62) (end 8.679 6.561) (width 0.2) (layer "B.Cu") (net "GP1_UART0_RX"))
 (segment (start -16.4616 -16.229) (end -17.7965 -16.229) (width 0.2) (layer "B.Cu") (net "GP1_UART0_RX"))
 (segment (start -17.7965 -16.229) (end -19.8745 -18.307) (width 0.2) (layer "B.Cu") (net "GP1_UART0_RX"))
 (segment (start -7.14 -8.89) (end -9.1226 -8.89) (width 0.2) (layer "B.Cu") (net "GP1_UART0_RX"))
 (segment (start -23.3117 -30.6217) (end -27.34 -34.65) (width 0.2) (layer "B.Cu") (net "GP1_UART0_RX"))
 (segment (start 8.679 -2.9852) (end 7.9781 -3.6861) (width 0.2) (layer "B.Cu") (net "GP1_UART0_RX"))
 (segment (start -19.8745 -20.6854) (end -23.3117 -24.1226) (width 0.2) (layer "B.Cu") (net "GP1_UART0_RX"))
 (segment (start -19.8745 -18.307) (end -19.8745 -20.6854) (width 0.2) (layer "B.Cu") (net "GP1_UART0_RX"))
 (segment (start -9.1226 -8.89) (end -16.4616 -16.229) (width 0.2) (layer "B.Cu") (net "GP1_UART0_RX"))
 (segment (start 7.2489 -3.6861) (end 2.2648 -8.6702) (width 0.2) (layer "B.Cu") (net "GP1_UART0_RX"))
 (segment (start -23.3117 -24.1226) (end -23.3117 -30.6217) (width 0.2) (layer "B.Cu") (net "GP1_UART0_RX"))
 (segment (start 7.9781 -3.6861) (end 7.2489 -3.6861) (width 0.2) (layer "B.Cu") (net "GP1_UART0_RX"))
 (segment (start -11.88 -2.54) (end -10.8231 -3.5969) (width 0.2) (layer "B.Cu") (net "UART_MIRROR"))
 (segment (start -10.8231 -3.5969) (end 4.0231 -3.5969) (width 0.2) (layer "B.Cu") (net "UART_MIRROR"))
 (segment (start 4.0231 -3.5969) (end 7.62 0) (width 0.2) (layer "B.Cu") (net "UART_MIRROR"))
 (segment (start -11.9189 -3.9884) (end 6.1716 -3.9884) (width 0.2) (layer "B.Cu") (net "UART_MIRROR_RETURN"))
 (segment (start -12.9671 -1.0871) (end -12.9671 -2.9402) (width 0.2) (layer "B.Cu") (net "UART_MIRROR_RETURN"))
 (segment (start -11.88 0) (end -12.9671 -1.0871) (width 0.2) (layer "B.Cu") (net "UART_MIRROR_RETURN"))
 (segment (start -12.9671 -2.9402) (end -11.9189 -3.9884) (width 0.2) (layer "B.Cu") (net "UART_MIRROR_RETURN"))
 (segment (start 6.1716 -3.9884) (end 7.62 -2.54) (width 0.2) (layer "B.Cu") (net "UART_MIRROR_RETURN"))
 (segment (start 7.62 -17.78) (end 2.2165 -12.3765) (width 0.2) (layer "B.Cu") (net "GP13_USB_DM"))
 (segment (start 2.2165 -12.3765) (end -2.8635 -12.3765) (width 0.2) (layer "B.Cu") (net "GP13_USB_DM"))
 (segment (start -2.8635 -12.3765) (end -5.08 -10.16) (width 0.2) (layer "B.Cu") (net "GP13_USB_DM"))
 (segment (start -5.4934 -9.0419) (end -3.6581 -9.0419) (width 0.2) (layer "B.Cu") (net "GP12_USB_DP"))
 (segment (start -17.78 -17.78) (end -13.7261 -17.78) (width 0.2) (layer "B.Cu") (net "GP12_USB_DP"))
 (segment (start -6.175 -10.2289) (end -6.175 -9.7235) (width 0.2) (layer "B.Cu") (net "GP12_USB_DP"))
 (segment (start -3.6581 -9.0419) (end -2.54 -10.16) (width 0.2) (layer "B.Cu") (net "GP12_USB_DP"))
 (segment (start -13.7261 -17.78) (end -6.175 -10.2289) (width 0.2) (layer "B.Cu") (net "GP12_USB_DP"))
 (segment (start -6.175 -9.7235) (end -5.4934 -9.0419) (width 0.2) (layer "B.Cu") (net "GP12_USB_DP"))
 (segment (start -7.62 -19.48) (end -7.62 -17.78) (width 0.2) (layer "F.Cu") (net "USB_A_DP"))
 (segment (start 1 -28.1) (end -7.62 -19.48) (width 0.2) (layer "F.Cu") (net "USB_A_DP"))
 (segment (start 15.5517 -28.499) (end 15.5517 -20.0083) (width 0.2) (layer "B.Cu") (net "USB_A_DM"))
 (segment (start -1 -28.1) (end 0.0147 -29.1147) (width 0.2) (layer "B.Cu") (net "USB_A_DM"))
 (segment (start 0.0147 -29.1147) (end 14.936 -29.1147) (width 0.2) (layer "B.Cu") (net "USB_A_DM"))
 (segment (start 14.936 -29.1147) (end 15.5517 -28.499) (width 0.2) (layer "B.Cu") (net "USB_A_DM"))
 (segment (start 15.5517 -20.0083) (end 17.78 -17.78) (width 0.2) (layer "B.Cu") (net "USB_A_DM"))
 (segment (start 14.5 -27.6) (end 14.5 -26.6483) (width 0.2) (layer "B.Cu") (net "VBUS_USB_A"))
 (segment (start 14.5 -26.6483) (end 11.4083 -26.6483) (width 0.2) (layer "B.Cu") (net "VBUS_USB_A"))
 (segment (start 11.4083 -26.6483) (end 2.54 -17.78) (width 0.2) (layer "B.Cu") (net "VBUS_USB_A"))
 (segment (start 16.1253 -29.4664) (end -2.1336 -29.4664) (width 0.2) (layer "B.Cu") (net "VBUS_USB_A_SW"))
 (segment (start 17.04 -28.5517) (end 16.1253 -29.4664) (width 0.2) (layer "B.Cu") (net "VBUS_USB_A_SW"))
 (segment (start -2.1336 -29.4664) (end -3.5 -28.1) (width 0.2) (layer "B.Cu") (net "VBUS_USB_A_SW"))
 (segment (start 17.04 -27.6) (end 17.04 -28.5517) (width 0.2) (layer "B.Cu") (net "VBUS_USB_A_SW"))
 (segment (start -24.8 -26.8983) (end -29.1569 -22.5414) (width 0.2) (layer "F.Cu") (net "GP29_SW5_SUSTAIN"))
 (segment (start -29.1569 0.5031) (end -27.12 2.54) (width 0.2) (layer "F.Cu") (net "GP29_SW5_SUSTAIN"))
 (segment (start -29.1569 -22.5414) (end -29.1569 0.5031) (width 0.2) (layer "F.Cu") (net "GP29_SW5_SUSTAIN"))
 (segment (start -24.8 -27.85) (end -24.8 -26.8983) (width 0.2) (layer "F.Cu") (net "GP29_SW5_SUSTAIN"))
 (segment (start -21.55 -16.35) (end -23.31 -14.59) (width 0.2) (layer "F.Cu") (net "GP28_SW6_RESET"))
 (segment (start -21.55 -20.85) (end -21.55 -16.35) (width 0.2) (layer "F.Cu") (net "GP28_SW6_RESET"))
 (segment (start -23.31 -3.81) (end -27.12 0) (width 0.2) (layer "F.Cu") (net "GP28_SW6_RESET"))
 (segment (start -23.31 -14.59) (end -23.31 -3.81) (width 0.2) (layer "F.Cu") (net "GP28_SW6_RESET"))
 (segment (start -20.1677 -32.5578) (end -20.1678 -32.5578) (width 0.2) (layer "F.Cu") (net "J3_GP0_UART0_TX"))
 (segment (start -20.1677 -18.4477) (end -20.1677 -32.5578) (width 0.2) (layer "F.Cu") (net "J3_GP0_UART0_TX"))
 (segment (start -11.88 10.16) (end -18.2299 3.8101) (width 0.2) (layer "F.Cu") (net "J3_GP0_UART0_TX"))
 (segment (start -18.2299 3.8101) (end -18.2299 -16.5099) (width 0.2) (layer "F.Cu") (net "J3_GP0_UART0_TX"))
 (segment (start -20.1678 -32.5578) (end -22.26 -34.65) (width 0.2) (layer "F.Cu") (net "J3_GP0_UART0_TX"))
 (segment (start -18.2299 -16.5099) (end -20.1677 -18.4477) (width 0.2) (layer "F.Cu") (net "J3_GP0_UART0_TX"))
 (segment (start -15.7231 -30.6531) (end -19.72 -34.65) (width 0.2) (layer "F.Cu") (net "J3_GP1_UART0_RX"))
 (segment (start -15.723 -30.6531) (end -15.7231 -30.6531) (width 0.2) (layer "F.Cu") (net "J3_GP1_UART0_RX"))
 (segment (start -11.88 7.62) (end -15.723 3.777) (width 0.2) (layer "F.Cu") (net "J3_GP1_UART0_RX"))
 (segment (start -15.723 3.777) (end -15.723 -30.6531) (width 0.2) (layer "F.Cu") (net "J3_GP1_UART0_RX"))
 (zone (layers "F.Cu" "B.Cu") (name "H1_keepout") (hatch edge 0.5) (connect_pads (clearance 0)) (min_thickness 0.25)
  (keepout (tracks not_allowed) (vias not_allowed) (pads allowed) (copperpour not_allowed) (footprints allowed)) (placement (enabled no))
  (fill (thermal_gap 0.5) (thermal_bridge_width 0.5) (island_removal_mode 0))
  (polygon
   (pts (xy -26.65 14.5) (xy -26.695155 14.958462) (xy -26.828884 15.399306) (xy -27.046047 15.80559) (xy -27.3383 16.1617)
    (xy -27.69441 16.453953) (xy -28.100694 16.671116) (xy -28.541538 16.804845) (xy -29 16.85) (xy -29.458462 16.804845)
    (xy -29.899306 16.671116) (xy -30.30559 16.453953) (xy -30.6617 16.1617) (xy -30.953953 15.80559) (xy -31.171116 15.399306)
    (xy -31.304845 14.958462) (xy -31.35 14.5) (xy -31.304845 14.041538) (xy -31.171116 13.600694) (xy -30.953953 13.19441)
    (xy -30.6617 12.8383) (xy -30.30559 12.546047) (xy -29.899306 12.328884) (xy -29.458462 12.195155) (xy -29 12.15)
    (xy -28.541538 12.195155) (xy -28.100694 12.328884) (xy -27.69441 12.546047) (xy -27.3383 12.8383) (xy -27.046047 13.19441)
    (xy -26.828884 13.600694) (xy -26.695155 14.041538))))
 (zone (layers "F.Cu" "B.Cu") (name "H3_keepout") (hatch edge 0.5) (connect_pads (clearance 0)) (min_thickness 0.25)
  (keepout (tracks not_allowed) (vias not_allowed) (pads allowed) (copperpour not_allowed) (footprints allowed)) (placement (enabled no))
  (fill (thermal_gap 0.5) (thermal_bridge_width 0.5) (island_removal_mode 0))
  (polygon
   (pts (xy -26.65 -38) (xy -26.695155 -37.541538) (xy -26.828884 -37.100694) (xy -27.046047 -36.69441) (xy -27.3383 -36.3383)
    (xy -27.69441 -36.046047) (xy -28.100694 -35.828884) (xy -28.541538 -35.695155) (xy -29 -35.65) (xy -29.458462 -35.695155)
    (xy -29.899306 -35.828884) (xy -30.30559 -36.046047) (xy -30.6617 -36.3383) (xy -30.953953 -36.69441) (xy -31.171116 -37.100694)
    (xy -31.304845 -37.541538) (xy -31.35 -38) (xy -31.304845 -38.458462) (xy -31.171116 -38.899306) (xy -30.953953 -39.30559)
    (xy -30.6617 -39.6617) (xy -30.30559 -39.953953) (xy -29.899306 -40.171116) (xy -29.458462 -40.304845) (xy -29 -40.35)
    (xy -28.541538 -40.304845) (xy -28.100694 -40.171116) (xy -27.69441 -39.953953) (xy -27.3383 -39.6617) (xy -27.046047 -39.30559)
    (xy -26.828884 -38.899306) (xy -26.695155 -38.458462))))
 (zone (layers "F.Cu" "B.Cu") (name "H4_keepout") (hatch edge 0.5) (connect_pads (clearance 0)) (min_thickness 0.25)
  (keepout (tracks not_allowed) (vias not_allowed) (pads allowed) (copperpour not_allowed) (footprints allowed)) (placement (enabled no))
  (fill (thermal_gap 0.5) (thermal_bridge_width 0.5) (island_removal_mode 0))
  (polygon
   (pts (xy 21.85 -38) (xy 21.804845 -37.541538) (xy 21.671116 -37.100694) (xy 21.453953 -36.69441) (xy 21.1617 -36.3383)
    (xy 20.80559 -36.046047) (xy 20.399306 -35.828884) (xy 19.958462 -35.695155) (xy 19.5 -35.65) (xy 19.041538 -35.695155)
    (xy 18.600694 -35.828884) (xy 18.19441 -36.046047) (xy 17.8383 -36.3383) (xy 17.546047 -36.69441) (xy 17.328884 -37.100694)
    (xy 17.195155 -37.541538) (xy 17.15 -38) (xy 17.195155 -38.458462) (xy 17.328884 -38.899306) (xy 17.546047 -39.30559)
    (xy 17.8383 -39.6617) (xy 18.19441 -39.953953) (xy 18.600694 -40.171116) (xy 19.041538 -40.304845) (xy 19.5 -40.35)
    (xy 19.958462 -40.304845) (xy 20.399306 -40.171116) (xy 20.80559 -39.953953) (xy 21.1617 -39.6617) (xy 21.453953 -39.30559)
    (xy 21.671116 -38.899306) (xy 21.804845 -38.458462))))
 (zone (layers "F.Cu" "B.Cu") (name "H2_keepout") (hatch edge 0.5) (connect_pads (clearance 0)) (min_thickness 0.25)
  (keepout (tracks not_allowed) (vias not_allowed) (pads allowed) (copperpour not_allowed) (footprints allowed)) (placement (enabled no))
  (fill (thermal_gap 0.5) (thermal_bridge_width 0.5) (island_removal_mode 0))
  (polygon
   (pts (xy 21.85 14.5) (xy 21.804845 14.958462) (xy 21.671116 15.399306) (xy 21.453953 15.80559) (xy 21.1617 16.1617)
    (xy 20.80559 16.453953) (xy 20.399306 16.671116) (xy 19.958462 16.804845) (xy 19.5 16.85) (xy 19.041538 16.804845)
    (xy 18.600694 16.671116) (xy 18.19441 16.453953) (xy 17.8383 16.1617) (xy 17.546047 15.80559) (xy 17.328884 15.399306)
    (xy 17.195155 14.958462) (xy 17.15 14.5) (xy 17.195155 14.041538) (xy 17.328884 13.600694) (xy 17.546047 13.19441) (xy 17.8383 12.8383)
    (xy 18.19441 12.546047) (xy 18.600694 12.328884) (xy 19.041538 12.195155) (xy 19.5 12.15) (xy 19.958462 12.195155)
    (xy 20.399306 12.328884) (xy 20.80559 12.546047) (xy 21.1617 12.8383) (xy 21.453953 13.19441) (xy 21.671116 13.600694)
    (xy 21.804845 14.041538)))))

